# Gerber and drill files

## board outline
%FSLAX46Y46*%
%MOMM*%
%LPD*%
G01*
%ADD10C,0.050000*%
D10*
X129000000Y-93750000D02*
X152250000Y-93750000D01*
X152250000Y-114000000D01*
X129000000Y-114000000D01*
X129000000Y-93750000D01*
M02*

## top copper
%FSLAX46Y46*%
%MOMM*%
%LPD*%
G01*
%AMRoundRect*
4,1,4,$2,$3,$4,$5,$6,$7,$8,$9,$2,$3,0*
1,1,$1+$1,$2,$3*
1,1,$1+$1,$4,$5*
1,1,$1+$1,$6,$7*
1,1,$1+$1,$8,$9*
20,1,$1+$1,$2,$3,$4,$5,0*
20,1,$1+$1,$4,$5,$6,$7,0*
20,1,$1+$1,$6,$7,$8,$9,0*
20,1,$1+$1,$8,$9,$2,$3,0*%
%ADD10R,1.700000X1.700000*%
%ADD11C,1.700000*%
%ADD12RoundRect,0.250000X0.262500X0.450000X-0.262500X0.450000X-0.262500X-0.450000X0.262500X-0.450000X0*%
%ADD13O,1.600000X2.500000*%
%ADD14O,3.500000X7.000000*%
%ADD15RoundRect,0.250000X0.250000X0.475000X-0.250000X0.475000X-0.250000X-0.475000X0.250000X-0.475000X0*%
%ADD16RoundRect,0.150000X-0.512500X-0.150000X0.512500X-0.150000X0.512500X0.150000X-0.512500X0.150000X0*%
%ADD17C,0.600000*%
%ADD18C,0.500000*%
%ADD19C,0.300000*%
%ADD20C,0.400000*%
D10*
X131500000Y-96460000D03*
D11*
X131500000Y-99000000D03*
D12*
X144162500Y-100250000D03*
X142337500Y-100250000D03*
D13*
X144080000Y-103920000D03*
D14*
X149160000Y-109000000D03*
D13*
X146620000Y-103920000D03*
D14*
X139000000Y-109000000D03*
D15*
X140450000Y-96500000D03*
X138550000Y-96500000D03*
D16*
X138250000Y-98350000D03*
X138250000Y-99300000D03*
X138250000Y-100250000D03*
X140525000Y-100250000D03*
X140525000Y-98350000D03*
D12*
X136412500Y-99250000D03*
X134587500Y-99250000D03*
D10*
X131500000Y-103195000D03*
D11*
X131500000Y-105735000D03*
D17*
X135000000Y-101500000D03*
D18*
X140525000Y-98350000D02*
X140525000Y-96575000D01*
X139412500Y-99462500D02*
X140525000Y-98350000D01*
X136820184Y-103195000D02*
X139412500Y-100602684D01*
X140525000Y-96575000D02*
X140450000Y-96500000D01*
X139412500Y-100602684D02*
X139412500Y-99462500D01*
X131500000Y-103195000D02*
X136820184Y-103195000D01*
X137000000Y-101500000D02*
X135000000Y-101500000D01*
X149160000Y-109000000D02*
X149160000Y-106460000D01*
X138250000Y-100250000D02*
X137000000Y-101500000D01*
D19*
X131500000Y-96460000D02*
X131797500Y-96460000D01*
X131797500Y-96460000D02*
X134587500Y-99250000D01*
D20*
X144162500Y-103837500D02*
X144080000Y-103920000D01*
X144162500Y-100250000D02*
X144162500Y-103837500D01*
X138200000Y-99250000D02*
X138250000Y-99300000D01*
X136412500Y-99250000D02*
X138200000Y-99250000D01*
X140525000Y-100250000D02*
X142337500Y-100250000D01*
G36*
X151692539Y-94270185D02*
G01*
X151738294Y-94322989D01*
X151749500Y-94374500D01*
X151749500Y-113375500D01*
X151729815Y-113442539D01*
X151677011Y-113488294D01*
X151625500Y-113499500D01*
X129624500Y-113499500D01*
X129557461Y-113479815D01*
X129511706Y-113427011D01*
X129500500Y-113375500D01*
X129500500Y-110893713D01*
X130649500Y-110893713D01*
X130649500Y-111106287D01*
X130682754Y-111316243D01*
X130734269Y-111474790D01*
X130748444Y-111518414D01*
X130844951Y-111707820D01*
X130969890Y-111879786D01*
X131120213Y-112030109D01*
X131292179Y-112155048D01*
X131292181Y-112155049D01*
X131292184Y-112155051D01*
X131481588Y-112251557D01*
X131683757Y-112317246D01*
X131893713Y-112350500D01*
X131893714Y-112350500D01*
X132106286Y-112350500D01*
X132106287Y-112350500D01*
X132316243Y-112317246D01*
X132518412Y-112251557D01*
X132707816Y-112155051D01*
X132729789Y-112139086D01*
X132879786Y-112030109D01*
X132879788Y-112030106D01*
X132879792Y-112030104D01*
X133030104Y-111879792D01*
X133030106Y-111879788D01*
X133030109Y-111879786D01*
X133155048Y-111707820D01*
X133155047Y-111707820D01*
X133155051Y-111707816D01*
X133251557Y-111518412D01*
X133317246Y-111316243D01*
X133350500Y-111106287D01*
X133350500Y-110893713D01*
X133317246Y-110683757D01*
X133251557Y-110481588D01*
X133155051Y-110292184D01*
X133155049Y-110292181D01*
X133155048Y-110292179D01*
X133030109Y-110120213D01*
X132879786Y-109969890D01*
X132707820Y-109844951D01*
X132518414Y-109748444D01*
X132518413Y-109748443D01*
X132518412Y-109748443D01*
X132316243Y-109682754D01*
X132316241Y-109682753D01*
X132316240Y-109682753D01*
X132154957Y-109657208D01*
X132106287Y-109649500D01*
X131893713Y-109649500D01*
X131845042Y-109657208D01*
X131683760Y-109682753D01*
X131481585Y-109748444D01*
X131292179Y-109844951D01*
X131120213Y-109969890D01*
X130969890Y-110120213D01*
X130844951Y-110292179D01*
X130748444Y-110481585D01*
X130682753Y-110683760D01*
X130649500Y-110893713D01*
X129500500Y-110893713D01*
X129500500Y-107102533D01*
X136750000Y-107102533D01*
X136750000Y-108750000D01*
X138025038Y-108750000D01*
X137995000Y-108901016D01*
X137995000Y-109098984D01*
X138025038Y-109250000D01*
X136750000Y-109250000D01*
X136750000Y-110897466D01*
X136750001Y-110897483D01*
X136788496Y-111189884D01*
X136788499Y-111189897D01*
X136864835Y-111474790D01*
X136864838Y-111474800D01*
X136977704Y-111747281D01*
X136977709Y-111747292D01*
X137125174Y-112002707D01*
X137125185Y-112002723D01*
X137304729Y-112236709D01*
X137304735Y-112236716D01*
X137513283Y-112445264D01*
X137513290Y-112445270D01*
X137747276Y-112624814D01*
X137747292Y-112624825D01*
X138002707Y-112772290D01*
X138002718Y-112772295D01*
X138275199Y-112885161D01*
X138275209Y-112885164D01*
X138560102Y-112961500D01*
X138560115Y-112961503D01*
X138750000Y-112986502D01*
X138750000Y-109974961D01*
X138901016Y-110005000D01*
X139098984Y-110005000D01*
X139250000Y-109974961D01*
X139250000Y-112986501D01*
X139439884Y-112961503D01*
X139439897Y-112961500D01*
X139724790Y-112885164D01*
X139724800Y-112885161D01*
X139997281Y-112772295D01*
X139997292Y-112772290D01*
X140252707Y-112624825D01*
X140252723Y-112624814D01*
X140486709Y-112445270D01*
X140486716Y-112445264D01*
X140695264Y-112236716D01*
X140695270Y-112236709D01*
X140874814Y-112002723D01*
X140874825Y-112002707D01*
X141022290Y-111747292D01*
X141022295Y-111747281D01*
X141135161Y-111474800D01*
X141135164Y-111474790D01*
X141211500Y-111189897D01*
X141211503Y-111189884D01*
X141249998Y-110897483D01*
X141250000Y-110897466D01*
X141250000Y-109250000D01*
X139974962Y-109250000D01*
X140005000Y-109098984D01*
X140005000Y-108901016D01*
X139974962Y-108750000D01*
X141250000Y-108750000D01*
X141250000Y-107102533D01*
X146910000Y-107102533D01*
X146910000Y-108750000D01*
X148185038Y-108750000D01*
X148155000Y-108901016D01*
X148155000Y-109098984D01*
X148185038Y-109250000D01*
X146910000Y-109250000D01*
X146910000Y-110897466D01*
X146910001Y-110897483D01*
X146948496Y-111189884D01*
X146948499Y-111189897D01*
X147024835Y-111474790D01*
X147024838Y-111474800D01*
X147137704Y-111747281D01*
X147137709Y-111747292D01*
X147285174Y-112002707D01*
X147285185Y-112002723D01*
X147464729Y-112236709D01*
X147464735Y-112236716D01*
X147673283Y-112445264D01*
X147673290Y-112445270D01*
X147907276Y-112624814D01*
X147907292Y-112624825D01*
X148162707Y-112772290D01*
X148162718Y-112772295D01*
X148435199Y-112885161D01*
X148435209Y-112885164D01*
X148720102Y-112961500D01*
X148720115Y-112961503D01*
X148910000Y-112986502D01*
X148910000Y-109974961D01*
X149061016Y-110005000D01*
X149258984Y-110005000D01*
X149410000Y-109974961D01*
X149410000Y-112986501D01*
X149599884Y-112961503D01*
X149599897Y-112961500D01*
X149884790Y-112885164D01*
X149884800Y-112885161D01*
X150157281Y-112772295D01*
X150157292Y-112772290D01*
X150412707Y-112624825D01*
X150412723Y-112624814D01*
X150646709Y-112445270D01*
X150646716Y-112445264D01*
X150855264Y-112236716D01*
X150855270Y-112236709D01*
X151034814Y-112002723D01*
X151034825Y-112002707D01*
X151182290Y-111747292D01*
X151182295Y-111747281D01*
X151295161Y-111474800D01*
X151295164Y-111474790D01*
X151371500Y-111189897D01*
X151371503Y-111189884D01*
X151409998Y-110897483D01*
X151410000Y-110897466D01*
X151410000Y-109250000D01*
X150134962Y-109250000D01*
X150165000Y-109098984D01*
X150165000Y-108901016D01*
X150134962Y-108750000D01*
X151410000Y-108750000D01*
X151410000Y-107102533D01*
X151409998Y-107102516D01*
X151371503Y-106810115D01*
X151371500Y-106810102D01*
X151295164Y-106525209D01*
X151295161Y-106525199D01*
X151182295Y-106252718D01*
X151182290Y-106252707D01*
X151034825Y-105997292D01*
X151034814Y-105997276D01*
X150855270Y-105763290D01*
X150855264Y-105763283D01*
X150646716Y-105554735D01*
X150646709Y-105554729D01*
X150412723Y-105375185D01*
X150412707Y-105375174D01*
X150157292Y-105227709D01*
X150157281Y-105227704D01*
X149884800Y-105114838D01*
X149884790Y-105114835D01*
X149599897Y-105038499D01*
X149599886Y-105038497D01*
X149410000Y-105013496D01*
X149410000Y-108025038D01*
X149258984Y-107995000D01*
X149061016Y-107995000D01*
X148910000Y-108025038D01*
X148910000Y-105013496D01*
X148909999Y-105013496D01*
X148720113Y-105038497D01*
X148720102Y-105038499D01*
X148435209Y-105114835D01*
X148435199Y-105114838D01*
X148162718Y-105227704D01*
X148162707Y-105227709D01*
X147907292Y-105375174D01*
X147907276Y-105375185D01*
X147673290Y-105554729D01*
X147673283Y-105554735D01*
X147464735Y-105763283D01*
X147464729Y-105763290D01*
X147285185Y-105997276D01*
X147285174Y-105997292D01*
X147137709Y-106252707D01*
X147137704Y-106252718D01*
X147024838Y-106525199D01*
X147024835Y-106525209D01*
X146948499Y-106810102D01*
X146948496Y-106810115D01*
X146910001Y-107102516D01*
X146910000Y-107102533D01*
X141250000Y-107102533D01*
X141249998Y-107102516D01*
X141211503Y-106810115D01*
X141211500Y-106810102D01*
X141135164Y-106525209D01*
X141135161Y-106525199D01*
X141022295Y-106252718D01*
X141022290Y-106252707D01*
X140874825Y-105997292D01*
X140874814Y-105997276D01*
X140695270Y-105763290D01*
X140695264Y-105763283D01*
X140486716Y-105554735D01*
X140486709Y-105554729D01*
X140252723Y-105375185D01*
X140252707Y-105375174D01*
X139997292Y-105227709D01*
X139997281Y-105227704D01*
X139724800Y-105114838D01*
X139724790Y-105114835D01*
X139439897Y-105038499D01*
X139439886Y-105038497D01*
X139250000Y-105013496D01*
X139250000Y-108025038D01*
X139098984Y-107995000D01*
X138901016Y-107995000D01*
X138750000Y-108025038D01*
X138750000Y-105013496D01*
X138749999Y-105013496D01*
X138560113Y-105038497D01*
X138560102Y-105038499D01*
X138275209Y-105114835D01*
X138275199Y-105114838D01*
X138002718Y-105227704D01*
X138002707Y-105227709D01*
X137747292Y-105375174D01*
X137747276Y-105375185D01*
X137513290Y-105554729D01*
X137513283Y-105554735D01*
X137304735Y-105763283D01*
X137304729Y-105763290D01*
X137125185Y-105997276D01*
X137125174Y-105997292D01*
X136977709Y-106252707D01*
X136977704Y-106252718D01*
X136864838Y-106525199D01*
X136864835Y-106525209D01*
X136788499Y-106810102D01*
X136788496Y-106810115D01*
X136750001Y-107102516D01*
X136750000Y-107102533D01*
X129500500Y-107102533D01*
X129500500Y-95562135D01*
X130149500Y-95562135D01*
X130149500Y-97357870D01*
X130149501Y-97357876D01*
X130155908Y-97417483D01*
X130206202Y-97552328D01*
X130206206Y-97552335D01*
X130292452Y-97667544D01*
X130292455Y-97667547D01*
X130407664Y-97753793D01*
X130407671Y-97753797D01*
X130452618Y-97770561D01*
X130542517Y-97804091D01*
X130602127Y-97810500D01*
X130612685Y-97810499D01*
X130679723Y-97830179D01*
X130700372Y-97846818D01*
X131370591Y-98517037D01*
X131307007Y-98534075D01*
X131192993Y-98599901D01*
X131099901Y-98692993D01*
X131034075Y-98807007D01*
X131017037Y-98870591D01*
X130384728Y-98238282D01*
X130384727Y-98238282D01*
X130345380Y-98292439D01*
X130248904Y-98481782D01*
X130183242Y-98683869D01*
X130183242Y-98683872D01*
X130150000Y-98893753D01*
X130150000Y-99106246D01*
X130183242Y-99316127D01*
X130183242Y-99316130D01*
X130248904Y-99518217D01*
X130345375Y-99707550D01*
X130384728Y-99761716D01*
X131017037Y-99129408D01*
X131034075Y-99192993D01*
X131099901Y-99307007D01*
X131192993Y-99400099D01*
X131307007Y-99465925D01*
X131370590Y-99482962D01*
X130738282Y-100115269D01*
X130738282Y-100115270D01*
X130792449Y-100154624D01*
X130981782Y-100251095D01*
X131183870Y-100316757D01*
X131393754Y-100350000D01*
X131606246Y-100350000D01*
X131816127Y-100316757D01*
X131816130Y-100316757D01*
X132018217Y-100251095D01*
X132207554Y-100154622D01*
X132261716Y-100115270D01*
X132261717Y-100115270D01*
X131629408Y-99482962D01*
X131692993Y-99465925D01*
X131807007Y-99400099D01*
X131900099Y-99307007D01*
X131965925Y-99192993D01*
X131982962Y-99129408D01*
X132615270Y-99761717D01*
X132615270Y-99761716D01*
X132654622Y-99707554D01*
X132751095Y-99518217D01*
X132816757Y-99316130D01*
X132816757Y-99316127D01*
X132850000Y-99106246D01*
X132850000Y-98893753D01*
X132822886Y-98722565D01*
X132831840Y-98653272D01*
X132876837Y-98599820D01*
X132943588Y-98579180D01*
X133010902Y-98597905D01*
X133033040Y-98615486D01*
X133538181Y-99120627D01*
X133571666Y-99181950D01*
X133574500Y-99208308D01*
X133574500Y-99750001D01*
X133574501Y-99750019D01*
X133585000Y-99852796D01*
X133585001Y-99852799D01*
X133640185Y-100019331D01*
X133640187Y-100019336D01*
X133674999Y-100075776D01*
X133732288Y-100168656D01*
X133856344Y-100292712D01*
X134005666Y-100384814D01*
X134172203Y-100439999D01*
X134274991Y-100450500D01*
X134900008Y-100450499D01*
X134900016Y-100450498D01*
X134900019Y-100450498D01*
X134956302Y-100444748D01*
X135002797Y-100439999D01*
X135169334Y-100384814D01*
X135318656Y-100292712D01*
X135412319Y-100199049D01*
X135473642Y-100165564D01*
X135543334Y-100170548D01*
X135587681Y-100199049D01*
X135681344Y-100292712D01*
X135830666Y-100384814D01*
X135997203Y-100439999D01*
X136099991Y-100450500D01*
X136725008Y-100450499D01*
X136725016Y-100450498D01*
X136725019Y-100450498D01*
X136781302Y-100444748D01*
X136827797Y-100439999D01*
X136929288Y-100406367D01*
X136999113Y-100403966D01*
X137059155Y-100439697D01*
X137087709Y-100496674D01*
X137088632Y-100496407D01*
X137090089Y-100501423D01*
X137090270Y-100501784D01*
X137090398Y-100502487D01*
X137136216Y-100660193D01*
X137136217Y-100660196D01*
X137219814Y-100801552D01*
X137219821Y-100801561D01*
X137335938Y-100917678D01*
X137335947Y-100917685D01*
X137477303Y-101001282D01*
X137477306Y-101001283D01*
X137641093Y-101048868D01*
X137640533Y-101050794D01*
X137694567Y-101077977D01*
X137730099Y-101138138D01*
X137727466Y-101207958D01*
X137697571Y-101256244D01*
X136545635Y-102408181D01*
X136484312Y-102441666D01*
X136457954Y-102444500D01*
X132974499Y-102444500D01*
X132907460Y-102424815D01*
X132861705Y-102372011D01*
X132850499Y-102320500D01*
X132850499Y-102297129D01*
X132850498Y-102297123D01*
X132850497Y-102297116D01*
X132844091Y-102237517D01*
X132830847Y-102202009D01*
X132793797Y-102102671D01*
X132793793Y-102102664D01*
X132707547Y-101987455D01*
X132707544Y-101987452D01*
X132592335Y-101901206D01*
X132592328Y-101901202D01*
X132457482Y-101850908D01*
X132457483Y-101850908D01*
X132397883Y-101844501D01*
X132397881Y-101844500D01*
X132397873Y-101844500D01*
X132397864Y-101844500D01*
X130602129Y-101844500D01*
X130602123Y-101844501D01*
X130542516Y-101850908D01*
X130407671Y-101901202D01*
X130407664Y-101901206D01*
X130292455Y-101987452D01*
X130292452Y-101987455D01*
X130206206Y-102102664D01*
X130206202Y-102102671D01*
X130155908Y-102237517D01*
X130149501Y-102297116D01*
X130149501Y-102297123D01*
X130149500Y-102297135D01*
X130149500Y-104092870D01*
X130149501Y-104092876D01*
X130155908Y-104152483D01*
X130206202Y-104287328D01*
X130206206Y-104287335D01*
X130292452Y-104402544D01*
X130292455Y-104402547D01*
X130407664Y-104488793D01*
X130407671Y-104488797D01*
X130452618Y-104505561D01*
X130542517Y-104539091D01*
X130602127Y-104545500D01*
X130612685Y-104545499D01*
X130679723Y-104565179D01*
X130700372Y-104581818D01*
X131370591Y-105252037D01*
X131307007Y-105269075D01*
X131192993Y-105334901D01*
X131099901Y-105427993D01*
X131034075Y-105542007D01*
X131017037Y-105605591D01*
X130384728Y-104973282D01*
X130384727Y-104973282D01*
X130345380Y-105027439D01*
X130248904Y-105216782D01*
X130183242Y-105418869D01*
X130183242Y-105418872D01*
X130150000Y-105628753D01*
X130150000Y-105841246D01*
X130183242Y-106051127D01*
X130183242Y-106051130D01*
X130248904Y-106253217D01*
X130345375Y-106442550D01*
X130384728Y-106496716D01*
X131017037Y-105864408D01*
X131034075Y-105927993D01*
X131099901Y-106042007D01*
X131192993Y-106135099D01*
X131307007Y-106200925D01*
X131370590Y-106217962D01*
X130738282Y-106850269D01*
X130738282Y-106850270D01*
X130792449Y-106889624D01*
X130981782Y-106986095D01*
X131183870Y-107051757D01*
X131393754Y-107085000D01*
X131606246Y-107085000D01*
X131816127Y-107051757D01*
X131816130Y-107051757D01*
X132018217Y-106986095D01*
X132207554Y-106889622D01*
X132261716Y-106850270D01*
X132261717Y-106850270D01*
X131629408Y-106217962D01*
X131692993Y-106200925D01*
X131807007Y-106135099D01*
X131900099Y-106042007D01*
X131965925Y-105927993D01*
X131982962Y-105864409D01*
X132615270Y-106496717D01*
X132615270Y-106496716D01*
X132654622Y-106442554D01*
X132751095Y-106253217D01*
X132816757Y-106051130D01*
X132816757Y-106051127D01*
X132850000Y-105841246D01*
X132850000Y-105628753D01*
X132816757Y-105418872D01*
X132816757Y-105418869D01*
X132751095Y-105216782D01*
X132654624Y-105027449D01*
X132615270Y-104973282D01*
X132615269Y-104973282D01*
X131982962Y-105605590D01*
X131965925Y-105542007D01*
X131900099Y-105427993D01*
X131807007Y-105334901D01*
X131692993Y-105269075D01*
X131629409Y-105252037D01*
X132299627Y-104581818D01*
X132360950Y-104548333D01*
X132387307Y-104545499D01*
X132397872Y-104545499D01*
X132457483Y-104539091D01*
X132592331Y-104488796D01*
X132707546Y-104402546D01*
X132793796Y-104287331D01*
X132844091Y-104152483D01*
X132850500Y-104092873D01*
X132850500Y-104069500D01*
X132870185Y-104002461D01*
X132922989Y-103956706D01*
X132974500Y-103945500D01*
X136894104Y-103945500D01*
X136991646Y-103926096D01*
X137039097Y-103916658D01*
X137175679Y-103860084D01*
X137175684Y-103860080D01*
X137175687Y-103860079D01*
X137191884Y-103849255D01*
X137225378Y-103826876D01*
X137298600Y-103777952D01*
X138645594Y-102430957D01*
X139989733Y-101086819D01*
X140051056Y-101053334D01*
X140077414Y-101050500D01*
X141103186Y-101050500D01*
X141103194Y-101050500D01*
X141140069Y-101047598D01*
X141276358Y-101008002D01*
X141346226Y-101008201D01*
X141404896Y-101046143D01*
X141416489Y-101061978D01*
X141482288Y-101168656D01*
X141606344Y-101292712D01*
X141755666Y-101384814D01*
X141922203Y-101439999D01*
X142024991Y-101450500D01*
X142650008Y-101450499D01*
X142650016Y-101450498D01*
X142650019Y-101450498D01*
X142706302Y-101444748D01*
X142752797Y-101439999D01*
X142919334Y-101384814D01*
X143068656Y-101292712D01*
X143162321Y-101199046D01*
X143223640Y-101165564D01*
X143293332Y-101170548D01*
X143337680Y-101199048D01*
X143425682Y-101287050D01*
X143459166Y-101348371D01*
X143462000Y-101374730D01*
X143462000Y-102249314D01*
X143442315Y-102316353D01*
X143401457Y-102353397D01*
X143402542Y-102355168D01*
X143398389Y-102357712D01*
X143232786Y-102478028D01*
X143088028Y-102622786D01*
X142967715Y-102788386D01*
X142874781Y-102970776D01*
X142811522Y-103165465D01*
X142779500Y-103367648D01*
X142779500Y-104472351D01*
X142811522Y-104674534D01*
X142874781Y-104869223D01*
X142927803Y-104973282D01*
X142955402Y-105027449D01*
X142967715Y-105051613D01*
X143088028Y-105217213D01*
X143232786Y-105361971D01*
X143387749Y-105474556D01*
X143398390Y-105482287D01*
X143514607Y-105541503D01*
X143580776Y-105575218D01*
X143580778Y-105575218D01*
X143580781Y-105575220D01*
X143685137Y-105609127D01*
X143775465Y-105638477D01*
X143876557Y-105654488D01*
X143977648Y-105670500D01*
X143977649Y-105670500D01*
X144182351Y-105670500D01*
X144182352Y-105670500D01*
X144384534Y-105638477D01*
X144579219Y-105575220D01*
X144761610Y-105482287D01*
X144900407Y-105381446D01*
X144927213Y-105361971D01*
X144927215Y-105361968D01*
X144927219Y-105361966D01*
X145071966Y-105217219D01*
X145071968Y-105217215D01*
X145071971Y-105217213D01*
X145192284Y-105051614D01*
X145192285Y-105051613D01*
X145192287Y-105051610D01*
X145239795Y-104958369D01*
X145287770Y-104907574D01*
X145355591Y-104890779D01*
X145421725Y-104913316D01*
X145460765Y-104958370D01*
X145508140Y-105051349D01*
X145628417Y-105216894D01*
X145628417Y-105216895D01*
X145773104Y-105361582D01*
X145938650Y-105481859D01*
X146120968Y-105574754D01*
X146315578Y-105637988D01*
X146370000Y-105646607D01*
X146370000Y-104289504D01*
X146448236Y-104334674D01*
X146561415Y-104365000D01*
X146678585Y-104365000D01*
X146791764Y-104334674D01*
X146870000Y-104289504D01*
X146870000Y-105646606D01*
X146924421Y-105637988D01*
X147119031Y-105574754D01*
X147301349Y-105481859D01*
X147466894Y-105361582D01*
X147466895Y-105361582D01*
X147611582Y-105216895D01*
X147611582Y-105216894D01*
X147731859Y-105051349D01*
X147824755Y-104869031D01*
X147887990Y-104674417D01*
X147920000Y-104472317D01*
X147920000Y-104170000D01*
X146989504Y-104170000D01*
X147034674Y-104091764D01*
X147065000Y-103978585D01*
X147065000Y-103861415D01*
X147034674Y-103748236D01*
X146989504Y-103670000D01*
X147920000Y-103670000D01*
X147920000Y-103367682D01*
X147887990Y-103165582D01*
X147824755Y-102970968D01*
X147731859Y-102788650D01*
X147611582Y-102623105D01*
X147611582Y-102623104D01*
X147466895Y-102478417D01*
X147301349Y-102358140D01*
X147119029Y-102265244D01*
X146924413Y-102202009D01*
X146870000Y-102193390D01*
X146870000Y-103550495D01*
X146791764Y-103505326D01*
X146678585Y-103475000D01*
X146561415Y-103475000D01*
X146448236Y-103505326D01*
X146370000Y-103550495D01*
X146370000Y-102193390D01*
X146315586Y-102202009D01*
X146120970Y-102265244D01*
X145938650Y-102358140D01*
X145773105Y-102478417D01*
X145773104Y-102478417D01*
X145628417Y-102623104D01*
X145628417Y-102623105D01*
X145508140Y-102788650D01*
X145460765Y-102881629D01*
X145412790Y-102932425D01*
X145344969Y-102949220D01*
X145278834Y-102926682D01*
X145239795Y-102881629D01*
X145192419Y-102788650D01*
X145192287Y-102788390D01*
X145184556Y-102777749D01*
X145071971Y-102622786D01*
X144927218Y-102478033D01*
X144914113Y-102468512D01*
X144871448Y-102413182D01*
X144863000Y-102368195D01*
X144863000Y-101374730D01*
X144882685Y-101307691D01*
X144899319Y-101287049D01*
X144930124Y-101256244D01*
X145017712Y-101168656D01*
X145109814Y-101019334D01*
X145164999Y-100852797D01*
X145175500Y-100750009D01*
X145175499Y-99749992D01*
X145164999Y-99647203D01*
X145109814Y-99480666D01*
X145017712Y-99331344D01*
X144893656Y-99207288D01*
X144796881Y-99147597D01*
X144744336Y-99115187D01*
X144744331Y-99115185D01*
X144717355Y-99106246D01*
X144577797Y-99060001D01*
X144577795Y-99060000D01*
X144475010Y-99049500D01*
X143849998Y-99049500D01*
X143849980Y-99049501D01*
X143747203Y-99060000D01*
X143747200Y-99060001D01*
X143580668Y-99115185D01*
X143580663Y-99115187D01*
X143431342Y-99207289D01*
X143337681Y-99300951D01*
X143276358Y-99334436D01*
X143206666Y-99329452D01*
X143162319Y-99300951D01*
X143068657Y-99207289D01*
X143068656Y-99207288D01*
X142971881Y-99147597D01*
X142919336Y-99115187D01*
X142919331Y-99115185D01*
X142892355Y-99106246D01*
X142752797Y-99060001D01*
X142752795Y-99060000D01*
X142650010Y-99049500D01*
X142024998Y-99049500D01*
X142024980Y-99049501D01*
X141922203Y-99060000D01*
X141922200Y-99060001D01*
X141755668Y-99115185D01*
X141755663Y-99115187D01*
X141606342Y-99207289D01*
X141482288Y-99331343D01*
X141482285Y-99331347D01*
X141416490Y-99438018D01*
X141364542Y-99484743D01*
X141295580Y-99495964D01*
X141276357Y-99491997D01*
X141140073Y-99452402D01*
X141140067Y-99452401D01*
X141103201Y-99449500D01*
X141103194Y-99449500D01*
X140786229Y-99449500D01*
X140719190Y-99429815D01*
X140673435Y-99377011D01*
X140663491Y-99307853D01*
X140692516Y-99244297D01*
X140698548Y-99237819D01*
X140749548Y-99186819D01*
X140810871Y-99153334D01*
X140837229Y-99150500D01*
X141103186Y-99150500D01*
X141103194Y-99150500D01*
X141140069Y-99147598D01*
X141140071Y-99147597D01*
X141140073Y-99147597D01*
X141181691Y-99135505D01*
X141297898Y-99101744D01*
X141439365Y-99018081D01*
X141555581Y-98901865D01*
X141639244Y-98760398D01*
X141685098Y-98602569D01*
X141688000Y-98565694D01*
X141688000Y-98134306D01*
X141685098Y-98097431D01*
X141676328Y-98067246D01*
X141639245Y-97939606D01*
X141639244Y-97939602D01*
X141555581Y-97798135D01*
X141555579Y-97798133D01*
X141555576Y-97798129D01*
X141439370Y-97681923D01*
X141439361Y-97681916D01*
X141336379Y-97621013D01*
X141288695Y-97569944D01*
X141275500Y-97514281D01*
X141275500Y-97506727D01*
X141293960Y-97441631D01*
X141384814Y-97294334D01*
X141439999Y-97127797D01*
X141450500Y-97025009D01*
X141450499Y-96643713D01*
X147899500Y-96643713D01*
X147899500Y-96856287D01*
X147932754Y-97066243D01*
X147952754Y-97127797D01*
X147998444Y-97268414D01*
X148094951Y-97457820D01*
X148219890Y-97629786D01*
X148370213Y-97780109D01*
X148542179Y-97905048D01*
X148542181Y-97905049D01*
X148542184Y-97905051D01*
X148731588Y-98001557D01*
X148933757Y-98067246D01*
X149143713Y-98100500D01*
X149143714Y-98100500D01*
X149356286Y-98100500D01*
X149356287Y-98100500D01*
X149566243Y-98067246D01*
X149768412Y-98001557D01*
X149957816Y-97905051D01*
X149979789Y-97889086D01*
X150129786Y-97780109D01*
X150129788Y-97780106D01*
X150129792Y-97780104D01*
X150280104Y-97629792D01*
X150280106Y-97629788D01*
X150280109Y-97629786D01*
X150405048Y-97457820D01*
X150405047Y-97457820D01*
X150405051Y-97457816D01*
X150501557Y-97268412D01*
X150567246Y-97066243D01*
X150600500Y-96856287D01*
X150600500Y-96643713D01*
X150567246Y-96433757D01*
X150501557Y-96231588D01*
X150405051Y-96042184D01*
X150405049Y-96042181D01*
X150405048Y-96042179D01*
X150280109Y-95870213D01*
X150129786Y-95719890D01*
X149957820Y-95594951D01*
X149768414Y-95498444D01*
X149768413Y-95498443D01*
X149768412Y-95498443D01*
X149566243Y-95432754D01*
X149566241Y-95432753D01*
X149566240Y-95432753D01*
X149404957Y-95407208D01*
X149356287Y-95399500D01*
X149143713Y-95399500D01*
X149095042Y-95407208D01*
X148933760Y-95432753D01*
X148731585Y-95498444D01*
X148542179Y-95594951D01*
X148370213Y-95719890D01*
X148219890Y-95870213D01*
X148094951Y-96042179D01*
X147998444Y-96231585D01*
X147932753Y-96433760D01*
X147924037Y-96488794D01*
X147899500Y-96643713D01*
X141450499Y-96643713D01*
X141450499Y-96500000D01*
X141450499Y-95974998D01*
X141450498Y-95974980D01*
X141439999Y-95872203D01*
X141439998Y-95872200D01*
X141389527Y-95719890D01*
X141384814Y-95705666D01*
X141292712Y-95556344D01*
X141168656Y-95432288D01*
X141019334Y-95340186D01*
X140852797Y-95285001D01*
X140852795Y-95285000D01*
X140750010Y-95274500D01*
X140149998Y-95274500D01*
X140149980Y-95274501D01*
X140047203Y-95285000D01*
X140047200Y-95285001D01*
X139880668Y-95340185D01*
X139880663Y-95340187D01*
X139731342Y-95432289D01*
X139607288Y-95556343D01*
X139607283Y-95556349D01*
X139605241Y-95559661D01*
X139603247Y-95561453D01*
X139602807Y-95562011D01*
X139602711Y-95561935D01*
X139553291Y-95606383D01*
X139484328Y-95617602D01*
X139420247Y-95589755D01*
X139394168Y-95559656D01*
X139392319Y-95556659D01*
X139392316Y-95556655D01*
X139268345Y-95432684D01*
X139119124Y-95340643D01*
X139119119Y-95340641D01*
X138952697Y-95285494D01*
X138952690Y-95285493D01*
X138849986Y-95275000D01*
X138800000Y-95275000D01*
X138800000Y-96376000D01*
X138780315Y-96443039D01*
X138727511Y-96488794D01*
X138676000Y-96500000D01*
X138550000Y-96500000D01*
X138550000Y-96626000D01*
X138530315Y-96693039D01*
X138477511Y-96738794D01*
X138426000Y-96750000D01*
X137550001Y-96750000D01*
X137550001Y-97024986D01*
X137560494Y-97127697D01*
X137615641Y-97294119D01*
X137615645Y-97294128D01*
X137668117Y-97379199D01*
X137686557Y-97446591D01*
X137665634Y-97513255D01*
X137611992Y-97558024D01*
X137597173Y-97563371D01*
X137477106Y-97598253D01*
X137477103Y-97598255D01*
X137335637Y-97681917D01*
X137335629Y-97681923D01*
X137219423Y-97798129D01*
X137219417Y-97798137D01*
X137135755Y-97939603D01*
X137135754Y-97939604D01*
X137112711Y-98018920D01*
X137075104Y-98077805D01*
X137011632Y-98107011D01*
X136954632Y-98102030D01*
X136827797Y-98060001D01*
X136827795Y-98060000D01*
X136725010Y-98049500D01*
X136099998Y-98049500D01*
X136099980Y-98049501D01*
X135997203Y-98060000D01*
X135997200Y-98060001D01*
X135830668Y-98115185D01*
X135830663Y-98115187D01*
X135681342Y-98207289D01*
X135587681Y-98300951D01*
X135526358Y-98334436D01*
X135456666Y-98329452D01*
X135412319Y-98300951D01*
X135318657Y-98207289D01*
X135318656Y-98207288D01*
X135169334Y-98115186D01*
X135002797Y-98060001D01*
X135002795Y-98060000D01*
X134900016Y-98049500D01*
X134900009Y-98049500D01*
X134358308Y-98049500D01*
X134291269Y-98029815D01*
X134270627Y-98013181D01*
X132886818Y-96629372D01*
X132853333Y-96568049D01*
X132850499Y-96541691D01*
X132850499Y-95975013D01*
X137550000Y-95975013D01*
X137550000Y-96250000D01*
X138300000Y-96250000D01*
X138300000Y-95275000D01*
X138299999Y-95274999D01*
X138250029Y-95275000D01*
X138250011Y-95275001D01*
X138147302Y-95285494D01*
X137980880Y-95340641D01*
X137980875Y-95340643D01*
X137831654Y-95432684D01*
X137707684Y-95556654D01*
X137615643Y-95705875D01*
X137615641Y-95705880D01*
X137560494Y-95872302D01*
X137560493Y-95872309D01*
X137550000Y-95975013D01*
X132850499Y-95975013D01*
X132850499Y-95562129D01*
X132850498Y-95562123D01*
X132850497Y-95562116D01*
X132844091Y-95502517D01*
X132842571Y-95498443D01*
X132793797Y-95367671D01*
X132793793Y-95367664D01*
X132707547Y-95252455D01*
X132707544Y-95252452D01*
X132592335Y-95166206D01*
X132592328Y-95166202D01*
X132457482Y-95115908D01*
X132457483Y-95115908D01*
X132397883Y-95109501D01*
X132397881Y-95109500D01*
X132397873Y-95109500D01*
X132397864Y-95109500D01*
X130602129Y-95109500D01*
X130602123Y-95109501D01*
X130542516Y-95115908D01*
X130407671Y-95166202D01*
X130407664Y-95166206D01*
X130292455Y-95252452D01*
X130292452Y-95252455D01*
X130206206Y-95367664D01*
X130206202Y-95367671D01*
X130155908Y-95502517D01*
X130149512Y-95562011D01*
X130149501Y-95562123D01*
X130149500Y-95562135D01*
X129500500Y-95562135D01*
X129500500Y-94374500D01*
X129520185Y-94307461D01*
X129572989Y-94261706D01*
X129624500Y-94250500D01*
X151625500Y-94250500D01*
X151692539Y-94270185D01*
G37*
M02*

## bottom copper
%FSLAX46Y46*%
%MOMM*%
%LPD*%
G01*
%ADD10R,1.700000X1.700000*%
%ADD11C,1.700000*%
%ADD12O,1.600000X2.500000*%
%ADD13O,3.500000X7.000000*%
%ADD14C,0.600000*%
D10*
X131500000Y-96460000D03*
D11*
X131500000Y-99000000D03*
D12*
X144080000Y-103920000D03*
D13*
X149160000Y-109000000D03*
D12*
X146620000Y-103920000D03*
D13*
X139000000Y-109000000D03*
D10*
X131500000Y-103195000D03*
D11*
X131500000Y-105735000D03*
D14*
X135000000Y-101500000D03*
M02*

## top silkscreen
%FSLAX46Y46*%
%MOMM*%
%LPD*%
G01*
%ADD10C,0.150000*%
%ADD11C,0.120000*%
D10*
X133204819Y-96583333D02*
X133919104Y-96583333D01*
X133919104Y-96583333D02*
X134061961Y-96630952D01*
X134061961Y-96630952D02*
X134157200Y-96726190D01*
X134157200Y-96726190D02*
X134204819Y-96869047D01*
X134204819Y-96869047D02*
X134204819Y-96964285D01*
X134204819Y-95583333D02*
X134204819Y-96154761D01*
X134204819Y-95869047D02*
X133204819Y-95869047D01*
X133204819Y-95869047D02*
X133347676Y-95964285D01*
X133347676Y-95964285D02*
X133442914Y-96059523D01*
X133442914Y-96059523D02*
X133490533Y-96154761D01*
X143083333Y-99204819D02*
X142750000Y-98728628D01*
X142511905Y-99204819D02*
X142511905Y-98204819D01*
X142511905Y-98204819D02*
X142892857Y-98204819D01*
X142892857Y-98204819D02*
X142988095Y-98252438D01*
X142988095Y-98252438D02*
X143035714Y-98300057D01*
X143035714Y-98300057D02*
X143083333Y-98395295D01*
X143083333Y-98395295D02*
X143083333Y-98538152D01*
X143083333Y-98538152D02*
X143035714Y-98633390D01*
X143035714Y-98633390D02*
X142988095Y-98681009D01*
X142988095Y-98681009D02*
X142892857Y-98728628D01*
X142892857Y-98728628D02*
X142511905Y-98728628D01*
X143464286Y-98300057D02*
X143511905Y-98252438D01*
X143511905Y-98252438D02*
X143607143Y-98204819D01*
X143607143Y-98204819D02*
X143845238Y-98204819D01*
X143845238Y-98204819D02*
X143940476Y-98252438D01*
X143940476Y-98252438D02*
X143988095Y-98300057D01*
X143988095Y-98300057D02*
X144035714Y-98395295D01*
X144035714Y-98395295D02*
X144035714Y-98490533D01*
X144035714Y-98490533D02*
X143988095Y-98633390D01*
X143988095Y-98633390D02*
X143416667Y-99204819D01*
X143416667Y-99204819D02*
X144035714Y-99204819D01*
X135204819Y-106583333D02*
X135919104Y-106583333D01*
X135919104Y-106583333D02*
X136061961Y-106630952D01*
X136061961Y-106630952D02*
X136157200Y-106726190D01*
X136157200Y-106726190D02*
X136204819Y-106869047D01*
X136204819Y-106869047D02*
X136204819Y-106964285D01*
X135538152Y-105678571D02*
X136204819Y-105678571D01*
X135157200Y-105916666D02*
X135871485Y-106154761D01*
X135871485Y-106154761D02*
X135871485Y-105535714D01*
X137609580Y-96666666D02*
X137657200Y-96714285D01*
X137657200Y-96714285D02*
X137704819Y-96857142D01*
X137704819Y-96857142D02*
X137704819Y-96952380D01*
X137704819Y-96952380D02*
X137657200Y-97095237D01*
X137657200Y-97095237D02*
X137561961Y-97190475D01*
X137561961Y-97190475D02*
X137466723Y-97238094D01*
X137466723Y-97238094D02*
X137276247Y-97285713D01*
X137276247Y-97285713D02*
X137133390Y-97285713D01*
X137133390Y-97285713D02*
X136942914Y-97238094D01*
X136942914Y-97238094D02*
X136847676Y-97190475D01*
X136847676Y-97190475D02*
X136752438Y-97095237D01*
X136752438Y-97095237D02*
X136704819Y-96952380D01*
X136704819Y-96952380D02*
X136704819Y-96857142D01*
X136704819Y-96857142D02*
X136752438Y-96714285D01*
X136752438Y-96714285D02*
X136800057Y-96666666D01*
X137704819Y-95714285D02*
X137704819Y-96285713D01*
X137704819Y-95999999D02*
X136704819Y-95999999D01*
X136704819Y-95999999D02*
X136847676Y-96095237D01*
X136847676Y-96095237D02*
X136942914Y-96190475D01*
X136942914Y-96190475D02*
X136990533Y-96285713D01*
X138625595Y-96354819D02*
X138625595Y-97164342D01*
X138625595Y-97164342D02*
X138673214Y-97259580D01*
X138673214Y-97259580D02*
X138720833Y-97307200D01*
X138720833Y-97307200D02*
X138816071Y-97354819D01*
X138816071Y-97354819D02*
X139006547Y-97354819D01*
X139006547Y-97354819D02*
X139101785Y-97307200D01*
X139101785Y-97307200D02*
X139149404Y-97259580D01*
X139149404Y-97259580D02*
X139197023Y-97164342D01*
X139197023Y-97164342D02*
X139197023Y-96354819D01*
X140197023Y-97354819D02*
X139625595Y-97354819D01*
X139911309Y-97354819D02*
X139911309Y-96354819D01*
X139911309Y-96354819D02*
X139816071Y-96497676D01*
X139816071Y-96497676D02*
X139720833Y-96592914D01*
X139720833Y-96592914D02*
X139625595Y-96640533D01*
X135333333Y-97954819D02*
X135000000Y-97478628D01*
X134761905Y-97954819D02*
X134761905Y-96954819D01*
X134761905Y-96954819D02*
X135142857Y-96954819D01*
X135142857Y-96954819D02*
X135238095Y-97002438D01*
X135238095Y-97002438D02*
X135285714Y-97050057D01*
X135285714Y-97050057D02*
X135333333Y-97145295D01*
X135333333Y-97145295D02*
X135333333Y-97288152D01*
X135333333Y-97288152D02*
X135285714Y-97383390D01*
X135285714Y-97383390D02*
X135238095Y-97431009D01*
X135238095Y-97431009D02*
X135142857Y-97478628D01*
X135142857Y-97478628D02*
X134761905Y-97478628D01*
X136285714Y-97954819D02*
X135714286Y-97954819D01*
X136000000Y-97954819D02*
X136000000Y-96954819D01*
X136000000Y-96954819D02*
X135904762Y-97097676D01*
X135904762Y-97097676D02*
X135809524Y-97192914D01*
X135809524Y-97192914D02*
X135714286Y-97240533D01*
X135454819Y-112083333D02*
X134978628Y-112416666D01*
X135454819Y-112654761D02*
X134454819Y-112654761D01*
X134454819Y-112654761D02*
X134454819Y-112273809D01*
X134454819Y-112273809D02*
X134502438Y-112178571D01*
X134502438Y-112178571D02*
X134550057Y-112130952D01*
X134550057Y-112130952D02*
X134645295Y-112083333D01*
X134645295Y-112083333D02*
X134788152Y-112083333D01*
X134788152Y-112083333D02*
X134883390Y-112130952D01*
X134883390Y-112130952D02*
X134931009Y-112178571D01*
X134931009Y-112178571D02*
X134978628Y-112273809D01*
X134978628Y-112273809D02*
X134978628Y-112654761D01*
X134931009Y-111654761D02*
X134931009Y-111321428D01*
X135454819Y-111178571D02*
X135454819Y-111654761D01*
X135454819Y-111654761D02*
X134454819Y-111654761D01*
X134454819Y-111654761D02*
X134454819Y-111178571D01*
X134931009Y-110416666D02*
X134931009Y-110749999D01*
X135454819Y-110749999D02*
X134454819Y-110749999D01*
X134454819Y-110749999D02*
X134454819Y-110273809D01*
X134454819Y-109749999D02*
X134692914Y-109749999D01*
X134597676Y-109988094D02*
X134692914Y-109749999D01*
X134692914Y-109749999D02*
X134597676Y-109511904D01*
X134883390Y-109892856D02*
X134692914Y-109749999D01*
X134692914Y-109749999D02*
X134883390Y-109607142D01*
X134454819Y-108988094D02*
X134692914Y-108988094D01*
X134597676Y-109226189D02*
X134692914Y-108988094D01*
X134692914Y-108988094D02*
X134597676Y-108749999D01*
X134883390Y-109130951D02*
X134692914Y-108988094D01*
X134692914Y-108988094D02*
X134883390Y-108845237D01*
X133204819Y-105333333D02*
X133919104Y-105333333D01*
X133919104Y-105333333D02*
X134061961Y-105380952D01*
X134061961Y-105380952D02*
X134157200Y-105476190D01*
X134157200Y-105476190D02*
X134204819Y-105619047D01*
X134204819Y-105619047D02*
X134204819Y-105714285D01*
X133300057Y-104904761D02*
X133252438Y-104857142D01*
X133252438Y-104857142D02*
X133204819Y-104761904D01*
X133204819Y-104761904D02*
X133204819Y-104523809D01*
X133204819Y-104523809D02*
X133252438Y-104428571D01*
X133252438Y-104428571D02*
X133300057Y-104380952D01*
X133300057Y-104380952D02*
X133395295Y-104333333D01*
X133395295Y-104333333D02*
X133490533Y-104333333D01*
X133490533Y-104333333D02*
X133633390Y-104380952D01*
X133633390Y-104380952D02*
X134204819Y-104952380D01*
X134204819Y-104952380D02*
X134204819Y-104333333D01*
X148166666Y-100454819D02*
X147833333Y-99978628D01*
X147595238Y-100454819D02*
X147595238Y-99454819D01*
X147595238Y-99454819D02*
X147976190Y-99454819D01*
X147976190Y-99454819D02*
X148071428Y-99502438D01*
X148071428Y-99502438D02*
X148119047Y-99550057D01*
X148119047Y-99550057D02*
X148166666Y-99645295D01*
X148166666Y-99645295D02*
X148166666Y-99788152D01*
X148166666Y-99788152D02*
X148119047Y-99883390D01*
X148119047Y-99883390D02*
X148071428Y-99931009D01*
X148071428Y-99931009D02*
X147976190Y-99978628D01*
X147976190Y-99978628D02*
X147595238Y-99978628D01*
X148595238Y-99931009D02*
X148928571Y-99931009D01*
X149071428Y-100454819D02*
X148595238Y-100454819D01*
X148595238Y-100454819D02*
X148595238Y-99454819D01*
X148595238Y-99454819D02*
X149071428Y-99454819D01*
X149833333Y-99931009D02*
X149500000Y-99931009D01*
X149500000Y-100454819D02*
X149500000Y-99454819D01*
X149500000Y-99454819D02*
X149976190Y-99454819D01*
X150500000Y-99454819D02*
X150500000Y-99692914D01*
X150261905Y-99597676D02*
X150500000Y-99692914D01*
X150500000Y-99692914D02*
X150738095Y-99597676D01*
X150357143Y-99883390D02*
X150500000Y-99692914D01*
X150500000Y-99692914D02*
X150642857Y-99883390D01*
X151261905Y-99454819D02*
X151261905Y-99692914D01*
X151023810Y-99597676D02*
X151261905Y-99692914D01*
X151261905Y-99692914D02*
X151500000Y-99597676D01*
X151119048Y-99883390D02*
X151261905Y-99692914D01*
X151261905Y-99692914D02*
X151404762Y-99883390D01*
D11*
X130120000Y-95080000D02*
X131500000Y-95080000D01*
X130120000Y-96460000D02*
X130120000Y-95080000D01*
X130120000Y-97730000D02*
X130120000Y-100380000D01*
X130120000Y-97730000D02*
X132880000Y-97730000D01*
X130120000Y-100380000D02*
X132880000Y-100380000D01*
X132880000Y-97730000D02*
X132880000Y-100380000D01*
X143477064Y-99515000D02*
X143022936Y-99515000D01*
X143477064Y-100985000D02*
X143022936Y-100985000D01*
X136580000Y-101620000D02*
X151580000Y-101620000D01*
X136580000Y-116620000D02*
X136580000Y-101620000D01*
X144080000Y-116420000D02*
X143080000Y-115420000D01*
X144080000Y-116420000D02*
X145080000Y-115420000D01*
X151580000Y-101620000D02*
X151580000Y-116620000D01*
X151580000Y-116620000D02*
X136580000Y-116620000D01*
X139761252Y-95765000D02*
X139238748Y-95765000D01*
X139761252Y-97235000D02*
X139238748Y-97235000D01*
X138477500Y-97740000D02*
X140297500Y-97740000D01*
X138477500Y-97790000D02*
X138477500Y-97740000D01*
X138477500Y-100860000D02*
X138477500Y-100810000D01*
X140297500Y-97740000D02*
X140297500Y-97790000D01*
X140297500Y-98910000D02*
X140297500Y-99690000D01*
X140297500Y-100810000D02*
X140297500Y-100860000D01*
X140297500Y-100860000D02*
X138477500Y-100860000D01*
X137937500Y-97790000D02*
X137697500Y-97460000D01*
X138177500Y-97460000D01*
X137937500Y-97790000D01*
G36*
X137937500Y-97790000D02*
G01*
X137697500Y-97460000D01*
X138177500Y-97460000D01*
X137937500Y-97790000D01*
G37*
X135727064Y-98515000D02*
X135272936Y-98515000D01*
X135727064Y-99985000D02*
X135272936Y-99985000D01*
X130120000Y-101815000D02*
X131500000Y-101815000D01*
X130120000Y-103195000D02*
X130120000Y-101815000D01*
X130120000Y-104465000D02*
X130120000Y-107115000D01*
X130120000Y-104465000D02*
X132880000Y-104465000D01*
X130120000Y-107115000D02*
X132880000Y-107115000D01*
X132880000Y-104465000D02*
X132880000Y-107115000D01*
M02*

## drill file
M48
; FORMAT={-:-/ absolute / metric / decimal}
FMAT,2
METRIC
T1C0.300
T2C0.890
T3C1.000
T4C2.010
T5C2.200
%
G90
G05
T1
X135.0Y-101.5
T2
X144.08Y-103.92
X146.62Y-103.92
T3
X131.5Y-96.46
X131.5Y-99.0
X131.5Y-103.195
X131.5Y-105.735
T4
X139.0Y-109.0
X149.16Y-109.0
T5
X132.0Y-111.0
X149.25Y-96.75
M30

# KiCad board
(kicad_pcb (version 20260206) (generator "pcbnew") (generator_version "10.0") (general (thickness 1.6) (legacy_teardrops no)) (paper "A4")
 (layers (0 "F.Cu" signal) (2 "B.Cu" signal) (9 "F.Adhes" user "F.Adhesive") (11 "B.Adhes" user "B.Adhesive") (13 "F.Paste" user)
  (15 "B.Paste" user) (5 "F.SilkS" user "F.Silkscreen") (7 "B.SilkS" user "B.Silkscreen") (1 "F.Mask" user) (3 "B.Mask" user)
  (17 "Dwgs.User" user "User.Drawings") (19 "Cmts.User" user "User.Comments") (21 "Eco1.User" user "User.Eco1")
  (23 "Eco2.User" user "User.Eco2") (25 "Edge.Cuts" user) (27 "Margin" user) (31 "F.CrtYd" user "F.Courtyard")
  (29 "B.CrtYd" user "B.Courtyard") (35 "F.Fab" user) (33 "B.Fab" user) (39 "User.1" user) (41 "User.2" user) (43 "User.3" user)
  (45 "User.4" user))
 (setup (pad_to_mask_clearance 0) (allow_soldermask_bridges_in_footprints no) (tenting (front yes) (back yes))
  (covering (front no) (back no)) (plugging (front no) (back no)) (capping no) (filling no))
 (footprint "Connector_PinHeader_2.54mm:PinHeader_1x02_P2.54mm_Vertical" (layer "F.Cu") (at 131.5 96.46)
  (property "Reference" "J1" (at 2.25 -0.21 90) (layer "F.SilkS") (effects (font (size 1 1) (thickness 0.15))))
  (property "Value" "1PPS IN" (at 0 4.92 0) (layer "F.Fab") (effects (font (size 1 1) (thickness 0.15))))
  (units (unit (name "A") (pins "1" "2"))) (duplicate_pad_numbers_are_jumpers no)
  (fp_line (start -1.38 -1.38) (end 0 -1.38) (stroke (width 0.12) (type solid)) (layer "F.SilkS"))
  (fp_line (start -1.38 0) (end -1.38 -1.38) (stroke (width 0.12) (type solid)) (layer "F.SilkS"))
  (fp_line (start -1.38 1.27) (end -1.38 3.92) (stroke (width 0.12) (type solid)) (layer "F.SilkS"))
  (fp_line (start -1.38 1.27) (end 1.38 1.27) (stroke (width 0.12) (type solid)) (layer "F.SilkS"))
  (fp_line (start -1.38 3.92) (end 1.38 3.92) (stroke (width 0.12) (type solid)) (layer "F.SilkS"))
  (fp_line (start 1.38 1.27) (end 1.38 3.92) (stroke (width 0.12) (type solid)) (layer "F.SilkS"))
  (pad "1" thru_hole rect (at 0 0) (size 1.7 1.7) (drill 1) (layers "*.Cu" "*.Mask") (remove_unused_layers no) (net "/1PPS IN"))
  (pad "2" thru_hole circle (at 0 2.54) (size 1.7 1.7) (drill 1) (layers "*.Cu" "*.Mask") (remove_unused_layers no) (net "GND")))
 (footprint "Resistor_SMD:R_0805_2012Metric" (layer "F.Cu") (at 143.25 100.25 180)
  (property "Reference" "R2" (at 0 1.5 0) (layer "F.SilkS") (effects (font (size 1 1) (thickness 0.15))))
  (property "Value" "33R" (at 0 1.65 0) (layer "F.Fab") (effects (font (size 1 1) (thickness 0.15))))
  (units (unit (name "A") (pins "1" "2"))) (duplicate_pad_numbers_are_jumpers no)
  (fp_line (start -0.227064 0.735) (end 0.227064 0.735) (stroke (width 0.12) (type solid)) (layer "F.SilkS"))
  (fp_line (start -0.227064 -0.735) (end 0.227064 -0.735) (stroke (width 0.12) (type solid)) (layer "F.SilkS"))
  (pad "1" smd roundrect (at -0.9125 0 180) (size 1.025 1.4) (layers "F.Cu" "F.Mask" "F.Paste") (roundrect_rratio 0.243902)
   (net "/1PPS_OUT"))
  (pad "2" smd roundrect (at 0.9125 0 180) (size 1.025 1.4) (layers "F.Cu" "F.Mask" "F.Paste") (roundrect_rratio 0.243902)
   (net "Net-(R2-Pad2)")))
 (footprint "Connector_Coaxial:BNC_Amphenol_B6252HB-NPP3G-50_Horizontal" (layer "F.Cu") (at 144.08 103.92 180)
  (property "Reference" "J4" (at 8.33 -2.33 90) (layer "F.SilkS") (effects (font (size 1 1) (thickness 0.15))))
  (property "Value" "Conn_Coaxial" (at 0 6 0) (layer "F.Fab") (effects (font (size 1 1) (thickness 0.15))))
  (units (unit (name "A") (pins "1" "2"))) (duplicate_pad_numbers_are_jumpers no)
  (fp_line (start 7.5 2.3) (end -7.5 2.3) (stroke (width 0.12) (type solid)) (layer "F.SilkS"))
  (fp_line (start 7.5 -12.7) (end 7.5 2.3) (stroke (width 0.12) (type solid)) (layer "F.SilkS"))
  (fp_line (start 0 -12.5) (end 1 -11.5) (stroke (width 0.12) (type solid)) (layer "F.SilkS"))
  (fp_line (start 0 -12.5) (end -1 -11.5) (stroke (width 0.12) (type solid)) (layer "F.SilkS"))
  (fp_line (start -7.5 2.3) (end -7.5 -12.7) (stroke (width 0.12) (type solid)) (layer "F.SilkS"))
  (fp_line (start -7.5 -12.7) (end 7.5 -12.7) (stroke (width 0.12) (type solid)) (layer "F.SilkS"))
  (pad "1" thru_hole oval (at 0 0 180) (size 1.6 2.5) (drill 0.89) (layers "*.Cu" "*.Mask") (remove_unused_layers no) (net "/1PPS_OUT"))
  (pad "2" thru_hole oval (at -5.08 -5.08 180) (size 3.5 7) (drill 2.01) (layers "*.Cu" "*.Mask") (remove_unused_layers no) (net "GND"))
  (pad "2" thru_hole oval (at -2.54 0 180) (size 1.6 2.5) (drill 0.89) (layers "*.Cu" "*.Mask") (remove_unused_layers no) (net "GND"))
  (pad "2" thru_hole oval (at 5.08 -5.08 180) (size 3.5 7) (drill 2.01) (layers "*.Cu" "*.Mask") (remove_unused_layers no) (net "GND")))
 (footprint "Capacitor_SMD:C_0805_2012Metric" (layer "F.Cu") (at 139.5 96.5 180)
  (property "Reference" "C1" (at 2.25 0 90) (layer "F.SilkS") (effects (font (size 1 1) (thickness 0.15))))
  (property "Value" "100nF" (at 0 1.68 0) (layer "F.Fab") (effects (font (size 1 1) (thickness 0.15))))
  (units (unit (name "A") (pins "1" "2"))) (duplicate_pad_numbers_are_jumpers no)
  (fp_line (start -0.261252 0.735) (end 0.261252 0.735) (stroke (width 0.12) (type solid)) (layer "F.SilkS"))
  (fp_line (start -0.261252 -0.735) (end 0.261252 -0.735) (stroke (width 0.12) (type solid)) (layer "F.SilkS"))
  (pad "1" smd roundrect (at -0.95 0 180) (size 1 1.45) (layers "F.Cu" "F.Mask" "F.Paste") (roundrect_rratio 0.25) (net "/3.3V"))
  (pad "2" smd roundrect (at 0.95 0 180) (size 1 1.45) (layers "F.Cu" "F.Mask" "F.Paste") (roundrect_rratio 0.25) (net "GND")))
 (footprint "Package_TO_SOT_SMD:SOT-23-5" (layer "F.Cu") (at 139.3875 99.3)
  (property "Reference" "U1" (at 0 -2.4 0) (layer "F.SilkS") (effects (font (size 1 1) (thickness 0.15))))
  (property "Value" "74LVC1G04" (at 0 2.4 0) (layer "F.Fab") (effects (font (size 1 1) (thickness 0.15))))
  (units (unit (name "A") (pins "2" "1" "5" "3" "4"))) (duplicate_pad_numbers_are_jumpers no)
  (fp_line (start -0.91 -1.56) (end 0.91 -1.56) (stroke (width 0.12) (type solid)) (layer "F.SilkS"))
  (fp_line (start -0.91 -1.51) (end -0.91 -1.56) (stroke (width 0.12) (type solid)) (layer "F.SilkS"))
  (fp_line (start -0.91 1.56) (end -0.91 1.51) (stroke (width 0.12) (type solid)) (layer "F.SilkS"))
  (fp_line (start 0.91 -1.56) (end 0.91 -1.51) (stroke (width 0.12) (type solid)) (layer "F.SilkS"))
  (fp_line (start 0.91 -0.39) (end 0.91 0.39) (stroke (width 0.12) (type solid)) (layer "F.SilkS"))
  (fp_line (start 0.91 1.51) (end 0.91 1.56) (stroke (width 0.12) (type solid)) (layer "F.SilkS"))
  (fp_line (start 0.91 1.56) (end -0.91 1.56) (stroke (width 0.12) (type solid)) (layer "F.SilkS"))
  (fp_poly (pts (xy -1.45 -1.51) (xy -1.69 -1.84) (xy -1.21 -1.84)) (stroke (width 0.12) (type solid)) (fill yes) (layer "F.SilkS"))
  (pad "1" smd roundrect (at -1.1375 -0.95) (size 1.325 0.6) (layers "F.Cu" "F.Mask" "F.Paste") (roundrect_rratio 0.25)
   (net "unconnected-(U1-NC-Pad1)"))
  (pad "2" smd roundrect (at -1.1375 0) (size 1.325 0.6) (layers "F.Cu" "F.Mask" "F.Paste") (roundrect_rratio 0.25) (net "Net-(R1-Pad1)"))
  (pad "3" smd roundrect (at -1.1375 0.95) (size 1.325 0.6) (layers "F.Cu" "F.Mask" "F.Paste") (roundrect_rratio 0.25) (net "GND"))
  (pad "4" smd roundrect (at 1.1375 0.95) (size 1.325 0.6) (layers "F.Cu" "F.Mask" "F.Paste") (roundrect_rratio 0.25) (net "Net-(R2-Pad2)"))
  (pad "5" smd roundrect (at 1.1375 -0.95) (size 1.325 0.6) (layers "F.Cu" "F.Mask" "F.Paste") (roundrect_rratio 0.25) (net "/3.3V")))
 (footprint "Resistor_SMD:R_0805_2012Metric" (layer "F.Cu") (at 135.5 99.25 180)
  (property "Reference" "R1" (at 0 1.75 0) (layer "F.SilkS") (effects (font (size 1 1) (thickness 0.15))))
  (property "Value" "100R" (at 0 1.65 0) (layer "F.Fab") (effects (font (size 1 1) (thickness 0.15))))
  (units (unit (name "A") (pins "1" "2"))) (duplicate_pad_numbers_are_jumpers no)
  (fp_line (start -0.227064 0.735) (end 0.227064 0.735) (stroke (width 0.12) (type solid)) (layer "F.SilkS"))
  (fp_line (start -0.227064 -0.735) (end 0.227064 -0.735) (stroke (width 0.12) (type solid)) (layer "F.SilkS"))
  (pad "1" smd roundrect (at -0.9125 0 180) (size 1.025 1.4) (layers "F.Cu" "F.Mask" "F.Paste") (roundrect_rratio 0.243902)
   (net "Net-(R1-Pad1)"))
  (pad "2" smd roundrect (at 0.9125 0 180) (size 1.025 1.4) (layers "F.Cu" "F.Mask" "F.Paste") (roundrect_rratio 0.243902) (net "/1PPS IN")))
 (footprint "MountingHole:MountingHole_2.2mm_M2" (layer "F.Cu") (at 132 111)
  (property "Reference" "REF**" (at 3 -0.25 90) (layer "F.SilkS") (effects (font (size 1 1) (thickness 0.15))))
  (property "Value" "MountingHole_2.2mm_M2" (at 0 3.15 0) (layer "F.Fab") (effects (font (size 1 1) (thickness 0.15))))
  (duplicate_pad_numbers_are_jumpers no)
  (pad "" np_thru_hole circle (at 0 0) (size 2.2 2.2) (drill 2.2) (layers "*.Cu" "*.Mask")))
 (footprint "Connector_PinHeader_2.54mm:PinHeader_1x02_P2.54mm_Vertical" (layer "F.Cu") (at 131.5 103.195)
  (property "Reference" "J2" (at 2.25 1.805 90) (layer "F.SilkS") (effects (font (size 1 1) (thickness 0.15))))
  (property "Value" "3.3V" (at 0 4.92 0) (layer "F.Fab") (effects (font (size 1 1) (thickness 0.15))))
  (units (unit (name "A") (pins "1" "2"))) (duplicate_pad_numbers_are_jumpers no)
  (fp_line (start -1.38 -1.38) (end 0 -1.38) (stroke (width 0.12) (type solid)) (layer "F.SilkS"))
  (fp_line (start -1.38 0) (end -1.38 -1.38) (stroke (width 0.12) (type solid)) (layer "F.SilkS"))
  (fp_line (start -1.38 1.27) (end -1.38 3.92) (stroke (width 0.12) (type solid)) (layer "F.SilkS"))
  (fp_line (start -1.38 1.27) (end 1.38 1.27) (stroke (width 0.12) (type solid)) (layer "F.SilkS"))
  (fp_line (start -1.38 3.92) (end 1.38 3.92) (stroke (width 0.12) (type solid)) (layer "F.SilkS"))
  (fp_line (start 1.38 1.27) (end 1.38 3.92) (stroke (width 0.12) (type solid)) (layer "F.SilkS"))
  (pad "1" thru_hole rect (at 0 0) (size 1.7 1.7) (drill 1) (layers "*.Cu" "*.Mask") (remove_unused_layers no) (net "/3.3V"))
  (pad "2" thru_hole circle (at 0 2.54) (size 1.7 1.7) (drill 1) (layers "*.Cu" "*.Mask") (remove_unused_layers no) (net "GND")))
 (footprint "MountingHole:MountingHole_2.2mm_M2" (layer "F.Cu") (at 149.25 96.75)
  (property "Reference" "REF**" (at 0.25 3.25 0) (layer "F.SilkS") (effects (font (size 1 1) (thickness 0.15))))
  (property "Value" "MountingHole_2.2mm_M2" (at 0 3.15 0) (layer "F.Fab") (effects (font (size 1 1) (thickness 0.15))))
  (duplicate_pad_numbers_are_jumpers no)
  (pad "" np_thru_hole circle (at 0 0) (size 2.2 2.2) (drill 2.2) (layers "*.Cu" "*.Mask")))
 (gr_rect (start 129 93.75) (end 152.25 114) (stroke (width 0.05) (type default)) (fill no) (layer "Edge.Cuts"))
 (segment (start 140.525 98.35) (end 140.525 96.575) (width 0.5) (layer "F.Cu") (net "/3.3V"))
 (segment (start 139.4125 99.4625) (end 140.525 98.35) (width 0.5) (layer "F.Cu") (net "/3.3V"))
 (segment (start 136.820184 103.195) (end 139.4125 100.602684) (width 0.5) (layer "F.Cu") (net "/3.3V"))
 (segment (start 140.525 96.575) (end 140.45 96.5) (width 0.5) (layer "F.Cu") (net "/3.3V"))
 (segment (start 139.4125 100.602684) (end 139.4125 99.4625) (width 0.5) (layer "F.Cu") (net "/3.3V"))
 (segment (start 131.5 103.195) (end 136.820184 103.195) (width 0.5) (layer "F.Cu") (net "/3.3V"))
 (segment (start 137 101.5) (end 135 101.5) (width 0.5) (layer "F.Cu") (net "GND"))
 (segment (start 149.16 109) (end 149.16 106.46) (width 0.5) (layer "F.Cu") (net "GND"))
 (segment (start 138.25 100.25) (end 137 101.5) (width 0.5) (layer "F.Cu") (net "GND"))
 (via (at 135 101.5) (size 0.6) (drill 0.3) (layers "F.Cu" "B.Cu") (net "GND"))
 (segment (start 131.5 96.46) (end 131.7975 96.46) (width 0.3) (layer "F.Cu") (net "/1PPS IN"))
 (segment (start 131.7975 96.46) (end 134.5875 99.25) (width 0.3) (layer "F.Cu") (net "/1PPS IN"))
 (segment (start 144.1625 103.8375) (end 144.08 103.92) (width 0.4) (layer "F.Cu") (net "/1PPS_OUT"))
 (segment (start 144.1625 100.25) (end 144.1625 103.8375) (width 0.4) (layer "F.Cu") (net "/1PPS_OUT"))
 (segment (start 138.2 99.25) (end 138.25 99.3) (width 0.4) (layer "F.Cu") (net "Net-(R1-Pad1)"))
 (segment (start 136.4125 99.25) (end 138.2 99.25) (width 0.4) (layer "F.Cu") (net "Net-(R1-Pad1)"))
 (segment (start 140.525 100.25) (end 142.3375 100.25) (width 0.4) (layer "F.Cu") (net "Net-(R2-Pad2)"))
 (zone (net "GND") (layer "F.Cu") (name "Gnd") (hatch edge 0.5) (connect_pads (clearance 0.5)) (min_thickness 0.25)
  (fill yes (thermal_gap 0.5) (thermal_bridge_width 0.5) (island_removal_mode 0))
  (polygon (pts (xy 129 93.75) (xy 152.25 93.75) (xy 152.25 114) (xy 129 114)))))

